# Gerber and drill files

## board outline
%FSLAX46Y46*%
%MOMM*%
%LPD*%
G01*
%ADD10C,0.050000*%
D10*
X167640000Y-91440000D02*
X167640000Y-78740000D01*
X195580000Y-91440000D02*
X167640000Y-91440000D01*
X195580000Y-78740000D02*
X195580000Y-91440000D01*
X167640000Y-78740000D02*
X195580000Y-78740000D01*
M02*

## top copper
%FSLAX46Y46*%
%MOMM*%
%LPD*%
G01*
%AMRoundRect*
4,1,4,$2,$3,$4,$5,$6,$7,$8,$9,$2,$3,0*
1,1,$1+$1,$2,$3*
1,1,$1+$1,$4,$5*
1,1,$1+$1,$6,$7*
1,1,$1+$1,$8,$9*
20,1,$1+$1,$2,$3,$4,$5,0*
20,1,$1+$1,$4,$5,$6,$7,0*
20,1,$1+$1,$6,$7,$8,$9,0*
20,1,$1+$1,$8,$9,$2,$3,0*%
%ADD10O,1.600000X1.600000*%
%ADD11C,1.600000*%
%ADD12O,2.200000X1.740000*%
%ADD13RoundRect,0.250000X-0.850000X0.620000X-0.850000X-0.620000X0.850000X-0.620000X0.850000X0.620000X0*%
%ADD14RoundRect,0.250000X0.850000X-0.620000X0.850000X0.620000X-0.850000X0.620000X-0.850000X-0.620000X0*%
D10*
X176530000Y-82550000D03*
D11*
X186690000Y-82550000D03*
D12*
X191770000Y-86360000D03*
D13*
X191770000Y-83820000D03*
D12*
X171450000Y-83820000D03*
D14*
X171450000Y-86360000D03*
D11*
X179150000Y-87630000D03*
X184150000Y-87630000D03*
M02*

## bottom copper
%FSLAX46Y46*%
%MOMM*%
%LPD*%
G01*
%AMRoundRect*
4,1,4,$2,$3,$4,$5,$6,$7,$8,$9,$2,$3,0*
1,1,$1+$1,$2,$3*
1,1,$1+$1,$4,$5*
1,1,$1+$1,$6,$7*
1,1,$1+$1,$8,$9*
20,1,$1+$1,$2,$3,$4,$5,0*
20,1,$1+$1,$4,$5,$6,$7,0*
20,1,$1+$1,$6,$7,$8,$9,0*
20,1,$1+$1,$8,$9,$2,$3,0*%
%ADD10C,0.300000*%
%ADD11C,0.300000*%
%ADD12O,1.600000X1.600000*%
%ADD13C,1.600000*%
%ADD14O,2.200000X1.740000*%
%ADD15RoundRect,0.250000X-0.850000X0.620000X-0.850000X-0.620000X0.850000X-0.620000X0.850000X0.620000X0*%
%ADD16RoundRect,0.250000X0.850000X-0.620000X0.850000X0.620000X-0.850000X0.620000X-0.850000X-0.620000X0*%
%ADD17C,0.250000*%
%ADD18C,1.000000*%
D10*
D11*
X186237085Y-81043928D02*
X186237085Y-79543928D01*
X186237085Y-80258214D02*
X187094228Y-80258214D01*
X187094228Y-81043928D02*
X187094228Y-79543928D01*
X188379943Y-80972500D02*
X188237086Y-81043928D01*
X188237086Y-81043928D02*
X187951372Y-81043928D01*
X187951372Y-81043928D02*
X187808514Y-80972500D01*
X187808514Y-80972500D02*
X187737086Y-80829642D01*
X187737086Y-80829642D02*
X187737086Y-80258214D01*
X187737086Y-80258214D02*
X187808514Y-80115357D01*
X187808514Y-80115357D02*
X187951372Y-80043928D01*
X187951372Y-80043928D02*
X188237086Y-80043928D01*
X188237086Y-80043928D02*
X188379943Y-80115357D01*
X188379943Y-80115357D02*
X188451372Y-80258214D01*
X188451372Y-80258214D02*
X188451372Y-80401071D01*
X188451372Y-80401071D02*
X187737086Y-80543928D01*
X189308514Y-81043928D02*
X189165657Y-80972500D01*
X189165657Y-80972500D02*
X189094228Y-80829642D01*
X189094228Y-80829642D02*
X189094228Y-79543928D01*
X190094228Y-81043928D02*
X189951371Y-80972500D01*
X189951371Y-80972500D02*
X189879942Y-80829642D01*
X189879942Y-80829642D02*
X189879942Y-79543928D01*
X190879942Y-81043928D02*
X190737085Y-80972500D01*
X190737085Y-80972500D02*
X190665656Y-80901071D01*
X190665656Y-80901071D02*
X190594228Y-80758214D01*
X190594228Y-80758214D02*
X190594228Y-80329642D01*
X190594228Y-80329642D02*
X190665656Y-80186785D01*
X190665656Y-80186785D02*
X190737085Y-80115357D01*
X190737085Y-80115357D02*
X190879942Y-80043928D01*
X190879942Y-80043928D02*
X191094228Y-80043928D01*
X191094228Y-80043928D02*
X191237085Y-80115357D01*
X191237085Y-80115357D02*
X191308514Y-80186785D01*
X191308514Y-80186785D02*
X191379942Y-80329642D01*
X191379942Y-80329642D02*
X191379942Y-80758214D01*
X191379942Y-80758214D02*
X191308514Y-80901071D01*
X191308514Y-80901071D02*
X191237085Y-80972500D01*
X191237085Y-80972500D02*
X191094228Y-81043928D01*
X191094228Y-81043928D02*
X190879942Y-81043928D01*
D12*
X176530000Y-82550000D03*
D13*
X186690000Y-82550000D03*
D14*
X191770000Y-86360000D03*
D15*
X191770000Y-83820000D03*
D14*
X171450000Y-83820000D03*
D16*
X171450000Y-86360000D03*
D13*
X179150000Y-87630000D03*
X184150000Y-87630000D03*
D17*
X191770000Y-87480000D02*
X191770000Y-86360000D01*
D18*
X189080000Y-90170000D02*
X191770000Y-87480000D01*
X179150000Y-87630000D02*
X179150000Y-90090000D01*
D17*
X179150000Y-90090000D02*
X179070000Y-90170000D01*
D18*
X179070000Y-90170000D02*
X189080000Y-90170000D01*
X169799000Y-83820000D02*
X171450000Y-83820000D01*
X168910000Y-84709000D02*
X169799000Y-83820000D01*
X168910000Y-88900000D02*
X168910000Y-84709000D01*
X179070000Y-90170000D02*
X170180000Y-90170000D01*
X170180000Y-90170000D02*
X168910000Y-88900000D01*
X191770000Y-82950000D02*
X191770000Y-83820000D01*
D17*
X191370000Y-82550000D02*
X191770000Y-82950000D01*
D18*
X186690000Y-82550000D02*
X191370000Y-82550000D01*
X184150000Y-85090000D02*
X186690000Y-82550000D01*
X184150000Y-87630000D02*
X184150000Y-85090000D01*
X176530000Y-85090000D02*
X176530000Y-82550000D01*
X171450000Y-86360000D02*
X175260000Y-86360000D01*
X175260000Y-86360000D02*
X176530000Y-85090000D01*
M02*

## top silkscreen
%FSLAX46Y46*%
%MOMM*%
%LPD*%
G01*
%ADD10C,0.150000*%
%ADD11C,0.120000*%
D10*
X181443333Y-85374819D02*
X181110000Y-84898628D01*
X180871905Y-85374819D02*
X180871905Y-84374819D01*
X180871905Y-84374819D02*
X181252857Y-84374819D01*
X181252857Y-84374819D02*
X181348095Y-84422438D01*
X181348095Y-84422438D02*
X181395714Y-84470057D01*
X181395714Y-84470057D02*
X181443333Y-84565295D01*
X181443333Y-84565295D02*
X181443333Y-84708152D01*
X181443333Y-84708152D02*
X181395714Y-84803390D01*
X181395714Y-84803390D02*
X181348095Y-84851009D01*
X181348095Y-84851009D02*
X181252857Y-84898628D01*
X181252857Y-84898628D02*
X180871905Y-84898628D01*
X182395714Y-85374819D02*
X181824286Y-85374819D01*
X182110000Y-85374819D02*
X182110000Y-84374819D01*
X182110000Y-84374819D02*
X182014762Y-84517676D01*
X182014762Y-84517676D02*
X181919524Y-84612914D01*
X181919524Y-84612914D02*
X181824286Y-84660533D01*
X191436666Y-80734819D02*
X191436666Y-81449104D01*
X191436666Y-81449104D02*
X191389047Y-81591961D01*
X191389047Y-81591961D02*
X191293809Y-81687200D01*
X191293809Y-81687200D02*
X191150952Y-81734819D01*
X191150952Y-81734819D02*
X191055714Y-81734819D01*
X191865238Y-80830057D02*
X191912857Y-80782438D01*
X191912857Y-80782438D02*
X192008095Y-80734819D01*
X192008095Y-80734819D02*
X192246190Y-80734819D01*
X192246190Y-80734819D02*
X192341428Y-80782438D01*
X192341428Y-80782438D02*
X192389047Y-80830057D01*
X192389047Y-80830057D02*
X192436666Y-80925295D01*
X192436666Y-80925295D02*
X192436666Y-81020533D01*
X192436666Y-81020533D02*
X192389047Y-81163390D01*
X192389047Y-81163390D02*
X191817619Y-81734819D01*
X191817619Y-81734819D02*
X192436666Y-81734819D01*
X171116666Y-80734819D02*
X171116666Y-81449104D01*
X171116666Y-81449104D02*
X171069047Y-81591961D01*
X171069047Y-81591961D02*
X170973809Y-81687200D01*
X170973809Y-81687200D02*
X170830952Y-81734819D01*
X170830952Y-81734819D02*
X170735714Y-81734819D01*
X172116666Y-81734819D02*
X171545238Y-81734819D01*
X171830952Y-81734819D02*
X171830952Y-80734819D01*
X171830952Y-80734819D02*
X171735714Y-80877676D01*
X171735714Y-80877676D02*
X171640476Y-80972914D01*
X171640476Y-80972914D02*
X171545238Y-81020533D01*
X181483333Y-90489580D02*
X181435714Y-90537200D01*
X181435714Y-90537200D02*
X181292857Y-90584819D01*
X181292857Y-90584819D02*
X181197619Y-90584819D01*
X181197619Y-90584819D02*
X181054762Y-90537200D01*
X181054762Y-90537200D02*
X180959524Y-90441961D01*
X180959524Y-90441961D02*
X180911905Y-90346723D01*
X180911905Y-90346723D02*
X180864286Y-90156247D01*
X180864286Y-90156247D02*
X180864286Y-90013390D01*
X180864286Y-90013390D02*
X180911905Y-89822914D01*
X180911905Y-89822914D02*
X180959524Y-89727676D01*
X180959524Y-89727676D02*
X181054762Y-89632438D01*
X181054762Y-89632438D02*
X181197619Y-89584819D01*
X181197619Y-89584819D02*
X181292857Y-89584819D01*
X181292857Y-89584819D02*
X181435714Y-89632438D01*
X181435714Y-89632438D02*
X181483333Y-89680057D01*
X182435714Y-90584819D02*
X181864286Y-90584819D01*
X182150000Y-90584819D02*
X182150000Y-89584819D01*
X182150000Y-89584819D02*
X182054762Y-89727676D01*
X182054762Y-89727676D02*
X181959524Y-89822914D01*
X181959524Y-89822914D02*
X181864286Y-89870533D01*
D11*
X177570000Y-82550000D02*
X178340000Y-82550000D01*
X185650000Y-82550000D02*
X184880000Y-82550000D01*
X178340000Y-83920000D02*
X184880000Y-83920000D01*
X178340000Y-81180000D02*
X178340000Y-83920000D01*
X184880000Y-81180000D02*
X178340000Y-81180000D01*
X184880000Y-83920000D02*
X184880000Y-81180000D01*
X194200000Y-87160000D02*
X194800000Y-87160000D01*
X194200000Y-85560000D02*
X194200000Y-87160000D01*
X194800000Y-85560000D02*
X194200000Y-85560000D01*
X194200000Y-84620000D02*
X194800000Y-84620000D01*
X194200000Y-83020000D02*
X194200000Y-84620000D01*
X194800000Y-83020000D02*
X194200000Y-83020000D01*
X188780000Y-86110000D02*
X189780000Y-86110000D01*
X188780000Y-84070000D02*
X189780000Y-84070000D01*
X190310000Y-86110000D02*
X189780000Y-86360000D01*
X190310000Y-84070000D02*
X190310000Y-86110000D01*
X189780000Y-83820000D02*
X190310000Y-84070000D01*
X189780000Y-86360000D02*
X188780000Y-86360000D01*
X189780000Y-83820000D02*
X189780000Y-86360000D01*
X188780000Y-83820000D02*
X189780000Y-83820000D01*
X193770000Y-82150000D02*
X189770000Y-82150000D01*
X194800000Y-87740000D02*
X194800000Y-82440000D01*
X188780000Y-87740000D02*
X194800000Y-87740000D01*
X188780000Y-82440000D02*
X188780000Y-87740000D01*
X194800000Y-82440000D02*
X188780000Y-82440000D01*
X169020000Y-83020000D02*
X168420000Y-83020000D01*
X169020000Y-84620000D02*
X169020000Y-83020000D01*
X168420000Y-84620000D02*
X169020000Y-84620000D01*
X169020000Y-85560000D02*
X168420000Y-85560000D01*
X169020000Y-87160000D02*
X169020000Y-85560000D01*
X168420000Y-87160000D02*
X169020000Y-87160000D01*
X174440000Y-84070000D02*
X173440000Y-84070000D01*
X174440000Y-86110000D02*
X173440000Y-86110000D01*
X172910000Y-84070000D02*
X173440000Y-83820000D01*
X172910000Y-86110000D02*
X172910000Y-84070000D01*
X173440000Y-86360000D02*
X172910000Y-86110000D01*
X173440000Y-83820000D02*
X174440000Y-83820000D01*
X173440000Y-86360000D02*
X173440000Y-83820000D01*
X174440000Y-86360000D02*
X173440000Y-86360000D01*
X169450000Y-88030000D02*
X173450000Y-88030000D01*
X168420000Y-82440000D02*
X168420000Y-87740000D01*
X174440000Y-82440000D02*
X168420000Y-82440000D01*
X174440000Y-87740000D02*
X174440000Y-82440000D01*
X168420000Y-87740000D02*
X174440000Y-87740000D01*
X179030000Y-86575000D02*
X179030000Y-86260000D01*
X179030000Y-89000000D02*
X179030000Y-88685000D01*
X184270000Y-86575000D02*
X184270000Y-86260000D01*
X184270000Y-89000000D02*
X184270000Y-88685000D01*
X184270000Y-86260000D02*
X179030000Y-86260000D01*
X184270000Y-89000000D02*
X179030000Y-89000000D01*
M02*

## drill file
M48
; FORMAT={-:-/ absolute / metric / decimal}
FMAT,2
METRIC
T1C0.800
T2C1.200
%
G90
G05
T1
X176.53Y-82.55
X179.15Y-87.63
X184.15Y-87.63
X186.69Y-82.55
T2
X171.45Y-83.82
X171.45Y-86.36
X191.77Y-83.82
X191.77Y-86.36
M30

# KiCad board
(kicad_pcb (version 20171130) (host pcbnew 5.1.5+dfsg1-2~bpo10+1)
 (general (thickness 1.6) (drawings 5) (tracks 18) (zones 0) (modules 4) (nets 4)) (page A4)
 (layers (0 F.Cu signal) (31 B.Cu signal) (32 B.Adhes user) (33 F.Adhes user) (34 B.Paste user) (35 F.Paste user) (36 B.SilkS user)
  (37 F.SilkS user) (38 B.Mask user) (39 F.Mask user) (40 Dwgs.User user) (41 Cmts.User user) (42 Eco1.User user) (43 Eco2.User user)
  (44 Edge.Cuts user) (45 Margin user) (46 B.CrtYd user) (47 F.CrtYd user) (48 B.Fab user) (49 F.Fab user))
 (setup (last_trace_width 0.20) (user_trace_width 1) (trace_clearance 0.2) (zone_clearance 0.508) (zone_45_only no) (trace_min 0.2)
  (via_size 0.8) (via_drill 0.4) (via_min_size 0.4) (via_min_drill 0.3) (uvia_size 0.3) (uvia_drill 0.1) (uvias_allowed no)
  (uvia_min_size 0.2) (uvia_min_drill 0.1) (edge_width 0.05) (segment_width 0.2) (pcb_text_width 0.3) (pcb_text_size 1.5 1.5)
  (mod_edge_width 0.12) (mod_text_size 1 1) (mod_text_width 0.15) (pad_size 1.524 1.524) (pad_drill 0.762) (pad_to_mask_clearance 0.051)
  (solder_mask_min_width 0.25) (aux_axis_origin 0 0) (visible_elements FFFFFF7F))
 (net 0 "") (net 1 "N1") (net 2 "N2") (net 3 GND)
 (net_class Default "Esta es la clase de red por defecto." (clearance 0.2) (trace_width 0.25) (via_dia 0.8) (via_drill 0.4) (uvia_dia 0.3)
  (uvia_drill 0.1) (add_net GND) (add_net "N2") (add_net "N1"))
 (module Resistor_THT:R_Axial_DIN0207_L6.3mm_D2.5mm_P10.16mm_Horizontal (layer F.Cu) (at 186.69 82.55 180)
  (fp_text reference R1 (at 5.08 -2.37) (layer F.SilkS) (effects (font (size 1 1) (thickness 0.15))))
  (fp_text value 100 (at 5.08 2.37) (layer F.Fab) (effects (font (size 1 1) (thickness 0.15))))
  (fp_line (start 9.12 0) (end 8.35 0) (layer F.SilkS) (width 0.12))
  (fp_line (start 1.04 0) (end 1.81 0) (layer F.SilkS) (width 0.12))
  (fp_line (start 8.35 -1.37) (end 1.81 -1.37) (layer F.SilkS) (width 0.12))
  (fp_line (start 8.35 1.37) (end 8.35 -1.37) (layer F.SilkS) (width 0.12))
  (fp_line (start 1.81 1.37) (end 8.35 1.37) (layer F.SilkS) (width 0.12))
  (fp_line (start 1.81 -1.37) (end 1.81 1.37) (layer F.SilkS) (width 0.12))
  (pad 2 thru_hole oval (at 10.16 0 180) (size 1.6 1.6) (drill 0.8) (layers *.Cu *.Mask) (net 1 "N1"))
  (pad 1 thru_hole circle (at 0 0 180) (size 1.6 1.6) (drill 0.8) (layers *.Cu *.Mask) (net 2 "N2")))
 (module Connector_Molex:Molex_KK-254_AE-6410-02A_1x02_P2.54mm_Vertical (layer F.Cu) (at 191.77 83.82 270)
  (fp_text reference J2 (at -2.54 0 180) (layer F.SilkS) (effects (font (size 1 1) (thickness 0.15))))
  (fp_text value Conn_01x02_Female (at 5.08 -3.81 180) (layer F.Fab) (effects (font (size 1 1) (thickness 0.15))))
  (fp_line (start 3.34 -2.43) (end 3.34 -3.03) (layer F.SilkS) (width 0.12))
  (fp_line (start 1.74 -2.43) (end 3.34 -2.43) (layer F.SilkS) (width 0.12))
  (fp_line (start 1.74 -3.03) (end 1.74 -2.43) (layer F.SilkS) (width 0.12))
  (fp_line (start 0.8 -2.43) (end 0.8 -3.03) (layer F.SilkS) (width 0.12))
  (fp_line (start -0.8 -2.43) (end 0.8 -2.43) (layer F.SilkS) (width 0.12))
  (fp_line (start -0.8 -3.03) (end -0.8 -2.43) (layer F.SilkS) (width 0.12))
  (fp_line (start 2.29 2.99) (end 2.29 1.99) (layer F.SilkS) (width 0.12))
  (fp_line (start 0.25 2.99) (end 0.25 1.99) (layer F.SilkS) (width 0.12))
  (fp_line (start 2.29 1.46) (end 2.54 1.99) (layer F.SilkS) (width 0.12))
  (fp_line (start 0.25 1.46) (end 2.29 1.46) (layer F.SilkS) (width 0.12))
  (fp_line (start 0 1.99) (end 0.25 1.46) (layer F.SilkS) (width 0.12))
  (fp_line (start 2.54 1.99) (end 2.54 2.99) (layer F.SilkS) (width 0.12))
  (fp_line (start 0 1.99) (end 2.54 1.99) (layer F.SilkS) (width 0.12))
  (fp_line (start 0 2.99) (end 0 1.99) (layer F.SilkS) (width 0.12))
  (fp_line (start -1.67 -2) (end -1.67 2) (layer F.SilkS) (width 0.12))
  (fp_line (start 3.92 -3.03) (end -1.38 -3.03) (layer F.SilkS) (width 0.12))
  (fp_line (start 3.92 2.99) (end 3.92 -3.03) (layer F.SilkS) (width 0.12))
  (fp_line (start -1.38 2.99) (end 3.92 2.99) (layer F.SilkS) (width 0.12))
  (fp_line (start -1.38 -3.03) (end -1.38 2.99) (layer F.SilkS) (width 0.12))
  (pad 2 thru_hole oval (at 2.54 0 270) (size 1.74 2.2) (drill 1.2) (layers *.Cu *.Mask) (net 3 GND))
  (pad 1 thru_hole roundrect (at 0 0 270) (size 1.74 2.2) (drill 1.2) (layers *.Cu *.Mask) (roundrect_rratio 0.143678) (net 2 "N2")))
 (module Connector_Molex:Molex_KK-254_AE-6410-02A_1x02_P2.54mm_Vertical (layer F.Cu) (at 171.45 86.36 90)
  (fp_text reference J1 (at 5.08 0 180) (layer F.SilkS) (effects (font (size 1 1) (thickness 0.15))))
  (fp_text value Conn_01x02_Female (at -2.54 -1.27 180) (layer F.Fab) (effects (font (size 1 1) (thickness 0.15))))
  (fp_line (start 3.34 -2.43) (end 3.34 -3.03) (layer F.SilkS) (width 0.12))
  (fp_line (start 1.74 -2.43) (end 3.34 -2.43) (layer F.SilkS) (width 0.12))
  (fp_line (start 1.74 -3.03) (end 1.74 -2.43) (layer F.SilkS) (width 0.12))
  (fp_line (start 0.8 -2.43) (end 0.8 -3.03) (layer F.SilkS) (width 0.12))
  (fp_line (start -0.8 -2.43) (end 0.8 -2.43) (layer F.SilkS) (width 0.12))
  (fp_line (start -0.8 -3.03) (end -0.8 -2.43) (layer F.SilkS) (width 0.12))
  (fp_line (start 2.29 2.99) (end 2.29 1.99) (layer F.SilkS) (width 0.12))
  (fp_line (start 0.25 2.99) (end 0.25 1.99) (layer F.SilkS) (width 0.12))
  (fp_line (start 2.29 1.46) (end 2.54 1.99) (layer F.SilkS) (width 0.12))
  (fp_line (start 0.25 1.46) (end 2.29 1.46) (layer F.SilkS) (width 0.12))
  (fp_line (start 0 1.99) (end 0.25 1.46) (layer F.SilkS) (width 0.12))
  (fp_line (start 2.54 1.99) (end 2.54 2.99) (layer F.SilkS) (width 0.12))
  (fp_line (start 0 1.99) (end 2.54 1.99) (layer F.SilkS) (width 0.12))
  (fp_line (start 0 2.99) (end 0 1.99) (layer F.SilkS) (width 0.12))
  (fp_line (start -1.67 -2) (end -1.67 2) (layer F.SilkS) (width 0.12))
  (fp_line (start 3.92 -3.03) (end -1.38 -3.03) (layer F.SilkS) (width 0.12))
  (fp_line (start 3.92 2.99) (end 3.92 -3.03) (layer F.SilkS) (width 0.12))
  (fp_line (start -1.38 2.99) (end 3.92 2.99) (layer F.SilkS) (width 0.12))
  (fp_line (start -1.38 -3.03) (end -1.38 2.99) (layer F.SilkS) (width 0.12))
  (pad 2 thru_hole oval (at 2.54 0 90) (size 1.74 2.2) (drill 1.2) (layers *.Cu *.Mask) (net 3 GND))
  (pad 1 thru_hole roundrect (at 0 0 90) (size 1.74 2.2) (drill 1.2) (layers *.Cu *.Mask) (roundrect_rratio 0.143678) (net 1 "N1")))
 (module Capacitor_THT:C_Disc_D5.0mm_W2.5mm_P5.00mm (layer F.Cu) (at 184.15 87.63 180)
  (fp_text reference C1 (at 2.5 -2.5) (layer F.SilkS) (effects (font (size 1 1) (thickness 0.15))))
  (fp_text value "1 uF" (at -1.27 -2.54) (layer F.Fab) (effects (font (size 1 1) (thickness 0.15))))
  (fp_line (start 5.12 1.055) (end 5.12 1.37) (layer F.SilkS) (width 0.12))
  (fp_line (start 5.12 -1.37) (end 5.12 -1.055) (layer F.SilkS) (width 0.12))
  (fp_line (start -0.12 1.055) (end -0.12 1.37) (layer F.SilkS) (width 0.12))
  (fp_line (start -0.12 -1.37) (end -0.12 -1.055) (layer F.SilkS) (width 0.12))
  (fp_line (start -0.12 1.37) (end 5.12 1.37) (layer F.SilkS) (width 0.12))
  (fp_line (start -0.12 -1.37) (end 5.12 -1.37) (layer F.SilkS) (width 0.12))
  (pad 2 thru_hole circle (at 5 0 180) (size 1.6 1.6) (drill 0.8) (layers *.Cu *.Mask) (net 3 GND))
  (pad 1 thru_hole circle (at 0 0 180) (size 1.6 1.6) (drill 0.8) (layers *.Cu *.Mask) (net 2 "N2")))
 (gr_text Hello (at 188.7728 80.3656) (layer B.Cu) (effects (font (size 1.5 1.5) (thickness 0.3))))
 (gr_line (start 167.64 91.44) (end 167.64 78.74) (layer Edge.Cuts) (width 0.05))
 (gr_line (start 195.58 91.44) (end 167.64 91.44) (layer Edge.Cuts) (width 0.05))
 (gr_line (start 195.58 78.74) (end 195.58 91.44) (layer Edge.Cuts) (width 0.05))
 (gr_line (start 167.64 78.74) (end 195.58 78.74) (layer Edge.Cuts) (width 0.05))
 (segment (start 191.77 87.48) (end 191.77 86.36) (width 0.25) (layer B.Cu) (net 3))
 (segment (start 189.08 90.17) (end 191.77 87.48) (width 1) (layer B.Cu) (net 3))
 (segment (start 179.15 87.63) (end 179.15 90.09) (width 1) (layer B.Cu) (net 3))
 (segment (start 179.15 90.09) (end 179.07 90.17) (width 0.25) (layer B.Cu) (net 3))
 (segment (start 179.07 90.17) (end 189.08 90.17) (width 1) (layer B.Cu) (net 3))
 (segment (start 169.799 83.82) (end 171.45 83.82) (width 1) (layer B.Cu) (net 3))
 (segment (start 168.91 84.709) (end 169.799 83.82) (width 1) (layer B.Cu) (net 3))
 (segment (start 168.91 88.9) (end 168.91 84.709) (width 1) (layer B.Cu) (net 3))
 (segment (start 179.07 90.17) (end 170.18 90.17) (width 1) (layer B.Cu) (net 3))
 (segment (start 170.18 90.17) (end 168.91 88.9) (width 1) (layer B.Cu) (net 3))
 (segment (start 191.77 82.95) (end 191.77 83.82) (width 1) (layer B.Cu) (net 2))
 (segment (start 191.37 82.55) (end 191.77 82.95) (width 0.25) (layer B.Cu) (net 2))
 (segment (start 186.69 82.55) (end 191.37 82.55) (width 1) (layer B.Cu) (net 2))
 (segment (start 184.15 85.09) (end 186.69 82.55) (width 1) (layer B.Cu) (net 2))
 (segment (start 184.15 87.63) (end 184.15 85.09) (width 1) (layer B.Cu) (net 2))
 (segment (start 176.53 85.09) (end 176.53 82.55) (width 1) (layer B.Cu) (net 1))
 (segment (start 171.45 86.36) (end 175.26 86.36) (width 1) (layer B.Cu) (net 1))
 (segment (start 175.26 86.36) (end 176.53 85.09) (width 1) (layer B.Cu) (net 1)))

